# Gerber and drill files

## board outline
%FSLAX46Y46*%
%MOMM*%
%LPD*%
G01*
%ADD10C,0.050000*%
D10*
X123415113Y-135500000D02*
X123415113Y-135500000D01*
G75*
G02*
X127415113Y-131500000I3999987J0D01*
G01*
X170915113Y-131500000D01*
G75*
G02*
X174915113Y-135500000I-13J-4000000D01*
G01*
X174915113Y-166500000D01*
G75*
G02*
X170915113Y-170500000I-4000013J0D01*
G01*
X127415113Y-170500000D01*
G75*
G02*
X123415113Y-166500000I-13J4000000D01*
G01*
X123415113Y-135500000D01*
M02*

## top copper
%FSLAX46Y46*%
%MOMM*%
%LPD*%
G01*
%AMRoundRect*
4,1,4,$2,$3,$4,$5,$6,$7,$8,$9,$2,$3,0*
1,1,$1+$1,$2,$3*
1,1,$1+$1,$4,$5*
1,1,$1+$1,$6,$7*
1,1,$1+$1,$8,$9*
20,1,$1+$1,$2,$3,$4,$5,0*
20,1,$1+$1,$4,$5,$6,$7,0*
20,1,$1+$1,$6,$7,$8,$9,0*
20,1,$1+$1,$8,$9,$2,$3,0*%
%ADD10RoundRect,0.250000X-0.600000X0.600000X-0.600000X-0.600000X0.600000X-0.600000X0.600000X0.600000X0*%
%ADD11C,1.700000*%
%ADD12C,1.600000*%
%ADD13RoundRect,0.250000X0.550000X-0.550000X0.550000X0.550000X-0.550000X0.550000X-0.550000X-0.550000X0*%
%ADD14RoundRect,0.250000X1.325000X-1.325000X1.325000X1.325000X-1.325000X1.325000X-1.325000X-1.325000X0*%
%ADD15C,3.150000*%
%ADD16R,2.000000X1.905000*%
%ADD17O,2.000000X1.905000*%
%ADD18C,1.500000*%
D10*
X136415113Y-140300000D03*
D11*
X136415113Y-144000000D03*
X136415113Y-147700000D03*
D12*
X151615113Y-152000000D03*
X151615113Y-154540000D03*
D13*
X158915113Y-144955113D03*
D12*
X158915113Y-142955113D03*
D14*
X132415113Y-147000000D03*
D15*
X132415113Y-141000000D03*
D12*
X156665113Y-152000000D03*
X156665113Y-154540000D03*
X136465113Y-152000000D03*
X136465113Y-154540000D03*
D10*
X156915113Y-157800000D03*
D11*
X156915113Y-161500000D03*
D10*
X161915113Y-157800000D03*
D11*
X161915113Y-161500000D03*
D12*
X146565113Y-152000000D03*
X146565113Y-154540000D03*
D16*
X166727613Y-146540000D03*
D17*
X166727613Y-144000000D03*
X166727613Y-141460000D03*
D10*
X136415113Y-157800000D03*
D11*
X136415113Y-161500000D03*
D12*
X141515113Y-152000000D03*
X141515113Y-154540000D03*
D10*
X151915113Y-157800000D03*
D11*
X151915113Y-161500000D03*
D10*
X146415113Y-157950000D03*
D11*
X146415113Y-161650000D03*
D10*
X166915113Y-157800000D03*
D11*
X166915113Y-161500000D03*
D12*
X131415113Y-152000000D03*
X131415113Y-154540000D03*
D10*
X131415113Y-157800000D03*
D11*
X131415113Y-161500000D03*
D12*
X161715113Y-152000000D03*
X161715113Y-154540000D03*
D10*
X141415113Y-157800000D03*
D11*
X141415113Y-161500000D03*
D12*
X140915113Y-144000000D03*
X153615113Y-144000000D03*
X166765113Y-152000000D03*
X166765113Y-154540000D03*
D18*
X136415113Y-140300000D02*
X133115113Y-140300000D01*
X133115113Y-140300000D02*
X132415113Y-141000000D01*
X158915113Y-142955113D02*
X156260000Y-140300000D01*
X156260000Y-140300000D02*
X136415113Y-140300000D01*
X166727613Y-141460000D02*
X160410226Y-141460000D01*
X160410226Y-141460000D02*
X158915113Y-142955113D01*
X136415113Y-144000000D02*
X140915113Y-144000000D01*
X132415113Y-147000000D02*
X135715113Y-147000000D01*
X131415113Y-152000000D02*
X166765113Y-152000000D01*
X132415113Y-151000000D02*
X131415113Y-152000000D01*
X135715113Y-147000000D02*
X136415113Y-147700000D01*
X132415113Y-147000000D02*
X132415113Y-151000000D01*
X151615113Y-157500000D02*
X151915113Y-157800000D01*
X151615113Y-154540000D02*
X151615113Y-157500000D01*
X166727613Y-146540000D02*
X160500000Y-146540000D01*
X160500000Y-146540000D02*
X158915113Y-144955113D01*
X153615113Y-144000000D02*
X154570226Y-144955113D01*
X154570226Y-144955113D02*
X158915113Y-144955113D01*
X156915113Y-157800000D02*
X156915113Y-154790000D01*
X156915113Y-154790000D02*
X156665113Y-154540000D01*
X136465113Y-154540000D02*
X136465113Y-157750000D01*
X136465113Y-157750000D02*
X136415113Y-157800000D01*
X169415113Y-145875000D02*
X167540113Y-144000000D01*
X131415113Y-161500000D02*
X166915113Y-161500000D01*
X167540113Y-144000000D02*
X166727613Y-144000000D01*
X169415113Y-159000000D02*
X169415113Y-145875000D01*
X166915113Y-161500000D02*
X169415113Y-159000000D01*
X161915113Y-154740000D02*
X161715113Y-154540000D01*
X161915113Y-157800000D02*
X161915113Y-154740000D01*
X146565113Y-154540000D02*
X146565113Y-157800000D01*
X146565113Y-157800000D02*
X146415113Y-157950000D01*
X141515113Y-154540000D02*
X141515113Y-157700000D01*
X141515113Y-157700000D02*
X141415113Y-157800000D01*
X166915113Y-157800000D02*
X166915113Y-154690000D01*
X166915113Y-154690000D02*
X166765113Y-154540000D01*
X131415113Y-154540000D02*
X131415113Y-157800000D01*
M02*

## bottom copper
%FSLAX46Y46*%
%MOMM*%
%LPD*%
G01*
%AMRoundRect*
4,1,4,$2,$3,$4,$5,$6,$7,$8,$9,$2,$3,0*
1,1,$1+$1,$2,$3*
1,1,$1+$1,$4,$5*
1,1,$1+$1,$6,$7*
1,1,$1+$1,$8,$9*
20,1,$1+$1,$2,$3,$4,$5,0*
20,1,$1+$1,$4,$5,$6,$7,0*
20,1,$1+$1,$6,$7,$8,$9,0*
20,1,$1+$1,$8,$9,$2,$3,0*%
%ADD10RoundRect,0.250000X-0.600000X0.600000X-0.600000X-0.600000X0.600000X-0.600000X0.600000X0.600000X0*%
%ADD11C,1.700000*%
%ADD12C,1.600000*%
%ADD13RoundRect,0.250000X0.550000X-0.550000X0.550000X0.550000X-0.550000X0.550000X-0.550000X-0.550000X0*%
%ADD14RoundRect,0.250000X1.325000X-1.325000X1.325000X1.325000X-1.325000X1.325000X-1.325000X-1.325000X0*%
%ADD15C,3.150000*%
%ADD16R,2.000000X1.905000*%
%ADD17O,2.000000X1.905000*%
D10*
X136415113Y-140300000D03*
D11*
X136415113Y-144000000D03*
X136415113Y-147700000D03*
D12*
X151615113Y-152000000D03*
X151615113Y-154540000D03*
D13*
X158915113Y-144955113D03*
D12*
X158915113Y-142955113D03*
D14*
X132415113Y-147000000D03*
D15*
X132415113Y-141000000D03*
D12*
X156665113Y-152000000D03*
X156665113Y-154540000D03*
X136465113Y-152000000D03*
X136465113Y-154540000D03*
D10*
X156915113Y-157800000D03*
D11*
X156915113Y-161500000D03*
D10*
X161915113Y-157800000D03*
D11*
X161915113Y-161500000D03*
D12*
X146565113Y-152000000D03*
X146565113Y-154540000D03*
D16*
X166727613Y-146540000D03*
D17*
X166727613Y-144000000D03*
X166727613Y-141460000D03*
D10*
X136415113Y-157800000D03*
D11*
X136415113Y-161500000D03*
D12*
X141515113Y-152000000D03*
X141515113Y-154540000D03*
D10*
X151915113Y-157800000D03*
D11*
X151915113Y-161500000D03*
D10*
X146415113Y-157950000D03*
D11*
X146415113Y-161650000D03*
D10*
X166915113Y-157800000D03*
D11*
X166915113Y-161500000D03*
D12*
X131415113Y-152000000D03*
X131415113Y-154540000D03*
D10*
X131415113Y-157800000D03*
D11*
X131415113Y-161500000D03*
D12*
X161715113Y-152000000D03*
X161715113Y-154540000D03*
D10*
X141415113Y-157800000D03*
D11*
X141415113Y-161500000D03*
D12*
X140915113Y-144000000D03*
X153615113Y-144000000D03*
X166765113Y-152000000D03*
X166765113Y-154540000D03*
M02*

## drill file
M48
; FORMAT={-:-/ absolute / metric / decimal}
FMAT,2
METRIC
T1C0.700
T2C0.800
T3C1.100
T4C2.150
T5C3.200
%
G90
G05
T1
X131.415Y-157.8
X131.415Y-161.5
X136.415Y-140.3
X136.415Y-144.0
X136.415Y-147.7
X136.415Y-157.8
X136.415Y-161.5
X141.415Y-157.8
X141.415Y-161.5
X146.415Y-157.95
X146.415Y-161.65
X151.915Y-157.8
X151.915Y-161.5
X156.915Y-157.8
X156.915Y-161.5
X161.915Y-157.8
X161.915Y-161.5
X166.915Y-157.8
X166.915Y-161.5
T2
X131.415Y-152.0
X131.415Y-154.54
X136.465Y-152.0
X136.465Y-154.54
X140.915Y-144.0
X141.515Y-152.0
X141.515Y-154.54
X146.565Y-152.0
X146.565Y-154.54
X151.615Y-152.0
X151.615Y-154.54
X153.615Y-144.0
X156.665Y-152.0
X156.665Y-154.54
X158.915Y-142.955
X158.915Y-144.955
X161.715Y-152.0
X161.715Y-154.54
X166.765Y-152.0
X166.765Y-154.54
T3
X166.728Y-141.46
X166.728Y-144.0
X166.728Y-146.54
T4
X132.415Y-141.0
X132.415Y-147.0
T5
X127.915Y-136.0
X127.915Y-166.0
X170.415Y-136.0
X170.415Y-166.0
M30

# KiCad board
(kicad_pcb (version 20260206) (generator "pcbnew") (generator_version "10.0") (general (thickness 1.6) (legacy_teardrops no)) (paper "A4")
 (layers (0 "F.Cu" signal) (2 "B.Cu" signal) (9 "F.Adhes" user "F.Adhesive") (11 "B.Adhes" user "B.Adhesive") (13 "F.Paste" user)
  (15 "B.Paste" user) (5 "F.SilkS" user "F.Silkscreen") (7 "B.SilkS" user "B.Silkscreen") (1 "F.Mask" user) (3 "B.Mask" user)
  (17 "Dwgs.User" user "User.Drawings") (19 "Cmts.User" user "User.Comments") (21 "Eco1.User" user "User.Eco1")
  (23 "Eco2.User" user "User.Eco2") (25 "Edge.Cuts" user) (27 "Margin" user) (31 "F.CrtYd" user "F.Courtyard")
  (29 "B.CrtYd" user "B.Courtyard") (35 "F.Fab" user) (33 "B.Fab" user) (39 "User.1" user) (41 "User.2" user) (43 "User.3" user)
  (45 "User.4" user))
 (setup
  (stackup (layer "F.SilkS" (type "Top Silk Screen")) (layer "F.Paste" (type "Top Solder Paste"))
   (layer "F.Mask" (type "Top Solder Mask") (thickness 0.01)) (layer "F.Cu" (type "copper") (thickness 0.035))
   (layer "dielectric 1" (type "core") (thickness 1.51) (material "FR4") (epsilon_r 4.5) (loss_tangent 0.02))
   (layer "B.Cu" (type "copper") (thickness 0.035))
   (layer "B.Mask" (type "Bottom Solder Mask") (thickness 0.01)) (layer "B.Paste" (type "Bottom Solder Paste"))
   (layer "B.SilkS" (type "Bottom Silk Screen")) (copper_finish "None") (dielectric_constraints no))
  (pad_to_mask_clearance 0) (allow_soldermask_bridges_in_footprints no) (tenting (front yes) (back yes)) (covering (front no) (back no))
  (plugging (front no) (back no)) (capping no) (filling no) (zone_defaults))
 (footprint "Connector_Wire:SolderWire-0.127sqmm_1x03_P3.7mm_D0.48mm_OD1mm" (layer "F.Cu") (at 136.415113 140.3 -90)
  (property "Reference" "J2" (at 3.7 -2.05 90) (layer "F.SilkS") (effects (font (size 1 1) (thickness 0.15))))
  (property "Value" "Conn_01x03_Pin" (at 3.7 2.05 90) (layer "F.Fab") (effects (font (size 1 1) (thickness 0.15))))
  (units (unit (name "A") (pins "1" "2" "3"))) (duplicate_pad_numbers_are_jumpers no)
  (pad "1" thru_hole roundrect (at 0 0 270) (size 1.7 1.7) (drill 0.7) (layers "*.Cu" "*.Mask") (remove_unused_layers no)
   (roundrect_rratio 0.147059) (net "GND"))
  (pad "2" thru_hole circle (at 3.7 0 270) (size 1.7 1.7) (drill 0.7) (layers "*.Cu" "*.Mask") (remove_unused_layers no)
   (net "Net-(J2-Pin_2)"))
  (pad "3" thru_hole circle (at 7.4 0 270) (size 1.7 1.7) (drill 0.7) (layers "*.Cu" "*.Mask") (remove_unused_layers no) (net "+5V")))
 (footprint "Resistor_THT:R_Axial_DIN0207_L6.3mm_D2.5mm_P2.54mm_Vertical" (layer "F.Cu") (at 151.615113 152 -90)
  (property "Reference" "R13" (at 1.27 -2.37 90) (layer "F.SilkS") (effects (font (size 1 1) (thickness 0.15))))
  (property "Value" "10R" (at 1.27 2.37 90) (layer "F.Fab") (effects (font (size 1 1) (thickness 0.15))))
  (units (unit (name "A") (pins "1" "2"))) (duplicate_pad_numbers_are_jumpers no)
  (pad "1" thru_hole circle (at 0 0 270) (size 1.6 1.6) (drill 0.8) (layers "*.Cu" "*.Mask") (remove_unused_layers no) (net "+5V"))
  (pad "2" thru_hole circle (at 2.54 0 270) (size 1.6 1.6) (drill 0.8) (layers "*.Cu" "*.Mask") (remove_unused_layers no)
   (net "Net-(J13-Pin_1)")))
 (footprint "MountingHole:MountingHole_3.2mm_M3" (layer "F.Cu") (at 170.415113 136)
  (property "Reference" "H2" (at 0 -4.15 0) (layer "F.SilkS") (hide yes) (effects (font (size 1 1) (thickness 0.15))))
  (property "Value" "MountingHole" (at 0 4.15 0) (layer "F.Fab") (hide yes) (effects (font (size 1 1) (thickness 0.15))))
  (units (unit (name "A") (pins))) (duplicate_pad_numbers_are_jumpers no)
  (pad "" np_thru_hole circle (at 0 0) (size 3.2 3.2) (drill 3.2) (layers "*.Cu" "*.Mask")))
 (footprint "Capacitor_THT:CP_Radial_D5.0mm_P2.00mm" (layer "F.Cu") (at 158.915113 144.955113 90)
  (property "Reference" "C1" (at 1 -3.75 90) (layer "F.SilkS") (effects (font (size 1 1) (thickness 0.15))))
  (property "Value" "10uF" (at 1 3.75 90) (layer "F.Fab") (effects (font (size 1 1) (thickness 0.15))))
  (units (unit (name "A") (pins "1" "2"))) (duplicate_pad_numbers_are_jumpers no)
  (pad "1" thru_hole roundrect (at 0 0 90) (size 1.6 1.6) (drill 0.8) (layers "*.Cu" "*.Mask") (remove_unused_layers no)
   (roundrect_rratio 0.15625) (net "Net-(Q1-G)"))
  (pad "2" thru_hole circle (at 2 0 90) (size 1.6 1.6) (drill 0.8) (layers "*.Cu" "*.Mask") (remove_unused_layers no) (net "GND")))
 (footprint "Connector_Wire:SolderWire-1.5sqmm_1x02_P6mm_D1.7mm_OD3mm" (layer "F.Cu") (at 132.415113 147 90)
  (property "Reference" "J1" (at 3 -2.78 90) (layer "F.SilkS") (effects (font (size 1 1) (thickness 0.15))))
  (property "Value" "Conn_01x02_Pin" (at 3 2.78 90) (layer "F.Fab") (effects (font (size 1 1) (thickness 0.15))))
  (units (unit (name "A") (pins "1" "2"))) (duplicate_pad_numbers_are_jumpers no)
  (pad "1" thru_hole roundrect (at 0 0 90) (size 3.15 3.15) (drill 2.15) (layers "*.Cu" "*.Mask") (remove_unused_layers no)
   (roundrect_rratio 0.079365) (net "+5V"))
  (pad "2" thru_hole circle (at 6 0 90) (size 3.15 3.15) (drill 2.15) (layers "*.Cu" "*.Mask") (remove_unused_layers no) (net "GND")))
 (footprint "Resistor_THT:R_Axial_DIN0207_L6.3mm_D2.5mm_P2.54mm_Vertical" (layer "F.Cu") (at 156.665113 152 -90)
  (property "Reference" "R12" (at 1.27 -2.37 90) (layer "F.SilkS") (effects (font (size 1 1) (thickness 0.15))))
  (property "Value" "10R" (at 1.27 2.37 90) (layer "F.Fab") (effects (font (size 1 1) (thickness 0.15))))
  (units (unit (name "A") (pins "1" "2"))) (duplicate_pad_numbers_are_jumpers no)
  (pad "1" thru_hole circle (at 0 0 270) (size 1.6 1.6) (drill 0.8) (layers "*.Cu" "*.Mask") (remove_unused_layers no) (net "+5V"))
  (pad "2" thru_hole circle (at 2.54 0 270) (size 1.6 1.6) (drill 0.8) (layers "*.Cu" "*.Mask") (remove_unused_layers no)
   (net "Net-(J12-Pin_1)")))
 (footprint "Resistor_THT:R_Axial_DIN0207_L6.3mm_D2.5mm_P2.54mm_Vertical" (layer "F.Cu") (at 136.465113 152 -90)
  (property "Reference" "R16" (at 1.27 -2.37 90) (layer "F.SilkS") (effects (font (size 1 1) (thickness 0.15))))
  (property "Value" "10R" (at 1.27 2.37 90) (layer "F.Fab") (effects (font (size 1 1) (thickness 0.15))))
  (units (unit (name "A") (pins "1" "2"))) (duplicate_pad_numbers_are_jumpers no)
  (pad "1" thru_hole circle (at 0 0 270) (size 1.6 1.6) (drill 0.8) (layers "*.Cu" "*.Mask") (remove_unused_layers no) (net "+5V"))
  (pad "2" thru_hole circle (at 2.54 0 270) (size 1.6 1.6) (drill 0.8) (layers "*.Cu" "*.Mask") (remove_unused_layers no)
   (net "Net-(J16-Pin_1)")))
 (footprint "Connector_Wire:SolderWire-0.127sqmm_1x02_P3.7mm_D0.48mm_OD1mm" (layer "F.Cu") (at 156.915113 157.8 -90)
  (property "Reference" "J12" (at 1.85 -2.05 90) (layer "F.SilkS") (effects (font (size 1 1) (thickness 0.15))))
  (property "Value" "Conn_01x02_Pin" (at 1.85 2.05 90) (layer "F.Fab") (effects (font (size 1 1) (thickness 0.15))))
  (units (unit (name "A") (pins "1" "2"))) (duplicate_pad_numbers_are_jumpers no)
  (pad "1" thru_hole roundrect (at 0 0 270) (size 1.7 1.7) (drill 0.7) (layers "*.Cu" "*.Mask") (remove_unused_layers no)
   (roundrect_rratio 0.147059) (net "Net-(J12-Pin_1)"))
  (pad "2" thru_hole circle (at 3.7 0 270) (size 1.7 1.7) (drill 0.7) (layers "*.Cu" "*.Mask") (remove_unused_layers no)
   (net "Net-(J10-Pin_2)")))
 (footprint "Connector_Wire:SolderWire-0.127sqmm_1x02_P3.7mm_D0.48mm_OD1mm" (layer "F.Cu") (at 161.915113 157.8 -90)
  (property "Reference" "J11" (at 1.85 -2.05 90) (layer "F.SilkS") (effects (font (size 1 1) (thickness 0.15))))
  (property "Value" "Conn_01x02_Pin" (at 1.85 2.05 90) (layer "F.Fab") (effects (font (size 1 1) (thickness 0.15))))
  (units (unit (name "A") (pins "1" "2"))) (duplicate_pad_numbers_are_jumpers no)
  (pad "1" thru_hole roundrect (at 0 0 270) (size 1.7 1.7) (drill 0.7) (layers "*.Cu" "*.Mask") (remove_unused_layers no)
   (roundrect_rratio 0.147059) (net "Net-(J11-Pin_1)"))
  (pad "2" thru_hole circle (at 3.7 0 270) (size 1.7 1.7) (drill 0.7) (layers "*.Cu" "*.Mask") (remove_unused_layers no)
   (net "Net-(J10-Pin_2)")))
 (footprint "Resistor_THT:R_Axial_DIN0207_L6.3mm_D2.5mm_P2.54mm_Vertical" (layer "F.Cu") (at 146.565113 152 -90)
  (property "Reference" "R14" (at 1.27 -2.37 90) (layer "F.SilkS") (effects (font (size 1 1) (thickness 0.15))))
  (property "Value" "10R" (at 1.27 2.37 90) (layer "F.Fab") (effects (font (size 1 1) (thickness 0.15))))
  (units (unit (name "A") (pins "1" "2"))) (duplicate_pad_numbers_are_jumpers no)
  (pad "1" thru_hole circle (at 0 0 270) (size 1.6 1.6) (drill 0.8) (layers "*.Cu" "*.Mask") (remove_unused_layers no) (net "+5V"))
  (pad "2" thru_hole circle (at 2.54 0 270) (size 1.6 1.6) (drill 0.8) (layers "*.Cu" "*.Mask") (remove_unused_layers no)
   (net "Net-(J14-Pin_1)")))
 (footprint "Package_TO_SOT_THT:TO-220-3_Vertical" (layer "F.Cu") (at 166.727613 146.54 90)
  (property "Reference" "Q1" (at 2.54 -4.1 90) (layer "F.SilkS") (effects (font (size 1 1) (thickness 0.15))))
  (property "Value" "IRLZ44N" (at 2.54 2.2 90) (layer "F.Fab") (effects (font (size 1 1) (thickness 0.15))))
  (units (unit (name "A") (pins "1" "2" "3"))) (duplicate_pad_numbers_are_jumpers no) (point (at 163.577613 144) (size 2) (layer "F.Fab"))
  (pad "1" thru_hole rect (at 0 0 90) (size 1.905 2) (drill 1.1) (layers "*.Cu" "*.Mask") (remove_unused_layers no) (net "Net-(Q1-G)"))
  (pad "2" thru_hole oval (at 2.54 0 90) (size 1.905 2) (drill 1.1) (layers "*.Cu" "*.Mask") (remove_unused_layers no)
   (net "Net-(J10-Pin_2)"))
  (pad "3" thru_hole oval (at 5.08 0 90) (size 1.905 2) (drill 1.1) (layers "*.Cu" "*.Mask") (remove_unused_layers no) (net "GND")))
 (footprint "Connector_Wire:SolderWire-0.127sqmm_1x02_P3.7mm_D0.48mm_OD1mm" (layer "F.Cu") (at 136.415113 157.8 -90)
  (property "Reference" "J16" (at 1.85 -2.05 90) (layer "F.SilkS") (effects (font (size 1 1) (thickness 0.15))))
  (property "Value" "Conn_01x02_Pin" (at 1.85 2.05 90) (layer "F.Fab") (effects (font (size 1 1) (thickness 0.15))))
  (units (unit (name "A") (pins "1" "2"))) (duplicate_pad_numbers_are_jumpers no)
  (pad "1" thru_hole roundrect (at 0 0 270) (size 1.7 1.7) (drill 0.7) (layers "*.Cu" "*.Mask") (remove_unused_layers no)
   (roundrect_rratio 0.147059) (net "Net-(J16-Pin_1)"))
  (pad "2" thru_hole circle (at 3.7 0 270) (size 1.7 1.7) (drill 0.7) (layers "*.Cu" "*.Mask") (remove_unused_layers no)
   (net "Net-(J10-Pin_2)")))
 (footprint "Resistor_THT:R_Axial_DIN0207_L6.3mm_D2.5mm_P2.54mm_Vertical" (layer "F.Cu") (at 141.515113 152 -90)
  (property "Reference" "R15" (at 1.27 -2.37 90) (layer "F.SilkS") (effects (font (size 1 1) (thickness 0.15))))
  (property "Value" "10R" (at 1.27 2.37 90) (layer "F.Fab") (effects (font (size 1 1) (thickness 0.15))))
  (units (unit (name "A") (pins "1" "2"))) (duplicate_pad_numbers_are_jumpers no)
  (pad "1" thru_hole circle (at 0 0 270) (size 1.6 1.6) (drill 0.8) (layers "*.Cu" "*.Mask") (remove_unused_layers no) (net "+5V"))
  (pad "2" thru_hole circle (at 2.54 0 270) (size 1.6 1.6) (drill 0.8) (layers "*.Cu" "*.Mask") (remove_unused_layers no)
   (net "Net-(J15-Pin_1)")))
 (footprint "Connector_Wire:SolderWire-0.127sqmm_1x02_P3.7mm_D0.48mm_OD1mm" (layer "F.Cu") (at 151.915113 157.8 -90)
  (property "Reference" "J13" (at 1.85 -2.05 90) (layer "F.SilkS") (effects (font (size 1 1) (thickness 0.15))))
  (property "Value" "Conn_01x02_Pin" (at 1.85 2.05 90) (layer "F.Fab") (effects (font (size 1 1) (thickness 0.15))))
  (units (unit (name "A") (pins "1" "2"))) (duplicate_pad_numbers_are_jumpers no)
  (pad "1" thru_hole roundrect (at 0 0 270) (size 1.7 1.7) (drill 0.7) (layers "*.Cu" "*.Mask") (remove_unused_layers no)
   (roundrect_rratio 0.147059) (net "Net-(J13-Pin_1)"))
  (pad "2" thru_hole circle (at 3.7 0 270) (size 1.7 1.7) (drill 0.7) (layers "*.Cu" "*.Mask") (remove_unused_layers no)
   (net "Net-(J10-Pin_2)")))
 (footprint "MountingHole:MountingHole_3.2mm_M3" (layer "F.Cu") (at 127.915113 136)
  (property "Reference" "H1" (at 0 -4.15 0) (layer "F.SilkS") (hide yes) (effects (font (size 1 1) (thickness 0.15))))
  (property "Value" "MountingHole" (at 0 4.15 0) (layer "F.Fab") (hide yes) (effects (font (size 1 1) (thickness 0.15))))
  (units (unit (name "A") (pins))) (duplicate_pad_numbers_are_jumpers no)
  (pad "" np_thru_hole circle (at 0 0) (size 3.2 3.2) (drill 3.2) (layers "*.Cu" "*.Mask")))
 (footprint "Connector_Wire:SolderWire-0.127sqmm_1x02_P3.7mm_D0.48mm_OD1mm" (layer "F.Cu") (at 146.415113 157.95 -90)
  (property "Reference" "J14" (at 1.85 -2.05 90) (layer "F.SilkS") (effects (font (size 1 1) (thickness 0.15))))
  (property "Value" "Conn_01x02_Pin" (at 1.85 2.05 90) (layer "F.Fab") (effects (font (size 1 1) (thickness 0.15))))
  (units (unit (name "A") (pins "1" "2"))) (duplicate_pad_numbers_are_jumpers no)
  (pad "1" thru_hole roundrect (at 0 0 270) (size 1.7 1.7) (drill 0.7) (layers "*.Cu" "*.Mask") (remove_unused_layers no)
   (roundrect_rratio 0.147059) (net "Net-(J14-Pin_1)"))
  (pad "2" thru_hole circle (at 3.7 0 270) (size 1.7 1.7) (drill 0.7) (layers "*.Cu" "*.Mask") (remove_unused_layers no)
   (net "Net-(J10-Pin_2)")))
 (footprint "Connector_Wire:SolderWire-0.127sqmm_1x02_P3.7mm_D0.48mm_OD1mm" (layer "F.Cu") (at 166.915113 157.8 -90)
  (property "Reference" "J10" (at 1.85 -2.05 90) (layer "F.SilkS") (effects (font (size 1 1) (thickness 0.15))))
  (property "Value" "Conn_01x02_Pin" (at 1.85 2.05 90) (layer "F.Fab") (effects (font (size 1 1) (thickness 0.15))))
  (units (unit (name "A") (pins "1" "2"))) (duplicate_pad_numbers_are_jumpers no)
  (pad "1" thru_hole roundrect (at 0 0 270) (size 1.7 1.7) (drill 0.7) (layers "*.Cu" "*.Mask") (remove_unused_layers no)
   (roundrect_rratio 0.147059) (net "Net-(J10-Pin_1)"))
  (pad "2" thru_hole circle (at 3.7 0 270) (size 1.7 1.7) (drill 0.7) (layers "*.Cu" "*.Mask") (remove_unused_layers no)
   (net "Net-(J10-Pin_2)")))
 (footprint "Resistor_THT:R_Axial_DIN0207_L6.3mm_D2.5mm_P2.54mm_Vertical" (layer "F.Cu") (at 131.415113 152 -90)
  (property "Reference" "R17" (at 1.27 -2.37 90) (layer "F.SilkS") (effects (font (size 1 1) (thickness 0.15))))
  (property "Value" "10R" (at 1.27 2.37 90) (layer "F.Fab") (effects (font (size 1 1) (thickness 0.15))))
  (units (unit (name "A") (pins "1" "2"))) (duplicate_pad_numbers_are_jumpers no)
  (pad "1" thru_hole circle (at 0 0 270) (size 1.6 1.6) (drill 0.8) (layers "*.Cu" "*.Mask") (remove_unused_layers no) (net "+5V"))
  (pad "2" thru_hole circle (at 2.54 0 270) (size 1.6 1.6) (drill 0.8) (layers "*.Cu" "*.Mask") (remove_unused_layers no)
   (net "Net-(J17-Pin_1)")))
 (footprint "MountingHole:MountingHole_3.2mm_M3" (layer "F.Cu") (at 127.915113 166)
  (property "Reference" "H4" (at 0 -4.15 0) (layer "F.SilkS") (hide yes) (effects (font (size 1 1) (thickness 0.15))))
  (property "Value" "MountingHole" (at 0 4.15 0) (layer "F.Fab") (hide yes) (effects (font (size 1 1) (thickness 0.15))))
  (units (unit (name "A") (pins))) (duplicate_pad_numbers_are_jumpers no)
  (pad "" np_thru_hole circle (at 0 0) (size 3.2 3.2) (drill 3.2) (layers "*.Cu" "*.Mask")))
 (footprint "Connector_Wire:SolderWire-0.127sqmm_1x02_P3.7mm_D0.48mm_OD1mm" (layer "F.Cu") (at 131.415113 157.8 -90)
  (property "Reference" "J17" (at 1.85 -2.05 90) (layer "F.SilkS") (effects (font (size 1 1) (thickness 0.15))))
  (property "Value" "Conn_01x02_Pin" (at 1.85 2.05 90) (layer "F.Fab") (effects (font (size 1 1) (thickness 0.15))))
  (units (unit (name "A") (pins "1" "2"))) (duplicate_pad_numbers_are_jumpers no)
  (pad "1" thru_hole roundrect (at 0 0 270) (size 1.7 1.7) (drill 0.7) (layers "*.Cu" "*.Mask") (remove_unused_layers no)
   (roundrect_rratio 0.147059) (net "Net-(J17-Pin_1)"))
  (pad "2" thru_hole circle (at 3.7 0 270) (size 1.7 1.7) (drill 0.7) (layers "*.Cu" "*.Mask") (remove_unused_layers no)
   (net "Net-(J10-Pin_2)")))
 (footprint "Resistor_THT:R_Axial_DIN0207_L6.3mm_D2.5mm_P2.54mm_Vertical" (layer "F.Cu") (at 161.715113 152 -90)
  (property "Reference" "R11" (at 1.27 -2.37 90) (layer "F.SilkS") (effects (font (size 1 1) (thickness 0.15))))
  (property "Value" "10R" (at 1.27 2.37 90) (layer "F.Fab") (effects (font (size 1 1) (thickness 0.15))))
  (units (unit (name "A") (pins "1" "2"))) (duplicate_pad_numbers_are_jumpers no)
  (pad "1" thru_hole circle (at 0 0 270) (size 1.6 1.6) (drill 0.8) (layers "*.Cu" "*.Mask") (remove_unused_layers no) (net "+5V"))
  (pad "2" thru_hole circle (at 2.54 0 270) (size 1.6 1.6) (drill 0.8) (layers "*.Cu" "*.Mask") (remove_unused_layers no)
   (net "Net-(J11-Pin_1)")))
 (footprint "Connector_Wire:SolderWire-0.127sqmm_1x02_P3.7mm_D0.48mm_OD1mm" (layer "F.Cu") (at 141.415113 157.8 -90)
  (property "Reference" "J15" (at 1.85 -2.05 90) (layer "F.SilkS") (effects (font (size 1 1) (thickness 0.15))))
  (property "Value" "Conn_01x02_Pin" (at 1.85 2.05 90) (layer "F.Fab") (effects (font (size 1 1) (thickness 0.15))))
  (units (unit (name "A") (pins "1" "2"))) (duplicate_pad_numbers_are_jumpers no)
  (pad "1" thru_hole roundrect (at 0 0 270) (size 1.7 1.7) (drill 0.7) (layers "*.Cu" "*.Mask") (remove_unused_layers no)
   (roundrect_rratio 0.147059) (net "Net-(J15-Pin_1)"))
  (pad "2" thru_hole circle (at 3.7 0 270) (size 1.7 1.7) (drill 0.7) (layers "*.Cu" "*.Mask") (remove_unused_layers no)
   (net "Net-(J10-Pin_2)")))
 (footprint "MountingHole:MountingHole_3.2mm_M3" (layer "F.Cu") (at 170.415113 166)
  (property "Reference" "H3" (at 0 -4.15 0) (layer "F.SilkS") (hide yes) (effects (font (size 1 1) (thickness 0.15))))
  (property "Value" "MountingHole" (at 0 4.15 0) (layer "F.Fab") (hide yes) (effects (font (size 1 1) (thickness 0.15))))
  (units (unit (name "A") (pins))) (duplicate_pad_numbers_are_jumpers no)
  (pad "" np_thru_hole circle (at 0 0) (size 3.2 3.2) (drill 3.2) (layers "*.Cu" "*.Mask")))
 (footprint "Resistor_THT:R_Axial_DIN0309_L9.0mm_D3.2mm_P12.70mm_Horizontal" (layer "F.Cu") (at 140.915113 144)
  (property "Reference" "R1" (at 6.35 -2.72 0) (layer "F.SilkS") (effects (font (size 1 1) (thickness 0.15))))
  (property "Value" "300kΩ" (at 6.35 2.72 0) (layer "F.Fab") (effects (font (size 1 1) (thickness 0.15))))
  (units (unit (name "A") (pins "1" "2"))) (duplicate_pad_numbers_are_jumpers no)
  (pad "1" thru_hole circle (at 0 0) (size 1.6 1.6) (drill 0.8) (layers "*.Cu" "*.Mask") (remove_unused_layers no) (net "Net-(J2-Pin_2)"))
  (pad "2" thru_hole circle (at 12.7 0) (size 1.6 1.6) (drill 0.8) (layers "*.Cu" "*.Mask") (remove_unused_layers no) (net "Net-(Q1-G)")))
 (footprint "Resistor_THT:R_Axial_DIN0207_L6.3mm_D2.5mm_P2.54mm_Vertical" (layer "F.Cu") (at 166.765113 152 -90)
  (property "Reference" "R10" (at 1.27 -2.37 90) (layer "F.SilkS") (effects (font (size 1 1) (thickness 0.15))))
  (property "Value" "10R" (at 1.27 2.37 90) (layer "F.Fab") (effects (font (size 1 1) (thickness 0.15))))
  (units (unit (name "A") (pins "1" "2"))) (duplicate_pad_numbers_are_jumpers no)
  (pad "1" thru_hole circle (at 0 0 270) (size 1.6 1.6) (drill 0.8) (layers "*.Cu" "*.Mask") (remove_unused_layers no) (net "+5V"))
  (pad "2" thru_hole circle (at 2.54 0 270) (size 1.6 1.6) (drill 0.8) (layers "*.Cu" "*.Mask") (remove_unused_layers no)
   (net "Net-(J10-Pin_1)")))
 (gr_rect (start 123.415113 131.5) (end 174.915113 170.5) (radius 4) (stroke (width 0.05) (type solid)) (fill no) (layer "Edge.Cuts"))
 (segment (start 136.415113 140.3) (end 133.115113 140.3) (width 1.5) (layer "F.Cu") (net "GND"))
 (segment (start 133.115113 140.3) (end 132.415113 141) (width 1.5) (layer "F.Cu") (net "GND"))
 (segment (start 158.915113 142.955113) (end 156.26 140.3) (width 1.5) (layer "F.Cu") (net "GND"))
 (segment (start 156.26 140.3) (end 136.415113 140.3) (width 1.5) (layer "F.Cu") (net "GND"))
 (segment (start 166.727613 141.46) (end 160.410226 141.46) (width 1.5) (layer "F.Cu") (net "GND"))
 (segment (start 160.410226 141.46) (end 158.915113 142.955113) (width 1.5) (layer "F.Cu") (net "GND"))
 (segment (start 136.415113 144) (end 140.915113 144) (width 1.5) (layer "F.Cu") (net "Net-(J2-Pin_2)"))
 (segment (start 132.415113 147) (end 135.715113 147) (width 1.5) (layer "F.Cu") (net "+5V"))
 (segment (start 131.415113 152) (end 166.765113 152) (width 1.5) (layer "F.Cu") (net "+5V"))
 (segment (start 132.415113 151) (end 131.415113 152) (width 1.5) (layer "F.Cu") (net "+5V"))
 (segment (start 135.715113 147) (end 136.415113 147.7) (width 1.5) (layer "F.Cu") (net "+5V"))
 (segment (start 132.415113 147) (end 132.415113 151) (width 1.5) (layer "F.Cu") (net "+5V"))
 (segment (start 151.615113 157.5) (end 151.915113 157.8) (width 1.5) (layer "F.Cu") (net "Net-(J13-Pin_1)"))
 (segment (start 151.615113 154.54) (end 151.615113 157.5) (width 1.5) (layer "F.Cu") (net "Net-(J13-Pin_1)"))
 (segment (start 166.727613 146.54) (end 160.5 146.54) (width 1.5) (layer "F.Cu") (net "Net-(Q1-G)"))
 (segment (start 160.5 146.54) (end 158.915113 144.955113) (width 1.5) (layer "F.Cu") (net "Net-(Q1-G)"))
 (segment (start 153.615113 144) (end 154.570226 144.955113) (width 1.5) (layer "F.Cu") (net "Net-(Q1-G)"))
 (segment (start 154.570226 144.955113) (end 158.915113 144.955113) (width 1.5) (layer "F.Cu") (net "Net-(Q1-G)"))
 (segment (start 156.915113 157.8) (end 156.915113 154.79) (width 1.5) (layer "F.Cu") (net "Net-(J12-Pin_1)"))
 (segment (start 156.915113 154.79) (end 156.665113 154.54) (width 1.5) (layer "F.Cu") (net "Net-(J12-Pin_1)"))
 (segment (start 136.465113 154.54) (end 136.465113 157.75) (width 1.5) (layer "F.Cu") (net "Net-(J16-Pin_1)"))
 (segment (start 136.465113 157.75) (end 136.415113 157.8) (width 1.5) (layer "F.Cu") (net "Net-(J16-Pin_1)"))
 (segment (start 169.415113 145.875) (end 167.540113 144) (width 1.5) (layer "F.Cu") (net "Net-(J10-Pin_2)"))
 (segment (start 131.415113 161.5) (end 166.915113 161.5) (width 1.5) (layer "F.Cu") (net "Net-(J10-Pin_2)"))
 (segment (start 167.540113 144) (end 166.727613 144) (width 1.5) (layer "F.Cu") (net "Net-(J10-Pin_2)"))
 (segment (start 169.415113 159) (end 169.415113 145.875) (width 1.5) (layer "F.Cu") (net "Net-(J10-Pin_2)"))
 (segment (start 166.915113 161.5) (end 169.415113 159) (width 1.5) (layer "F.Cu") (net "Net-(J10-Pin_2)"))
 (segment (start 161.915113 154.74) (end 161.715113 154.54) (width 1.5) (layer "F.Cu") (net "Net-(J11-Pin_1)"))
 (segment (start 161.915113 157.8) (end 161.915113 154.74) (width 1.5) (layer "F.Cu") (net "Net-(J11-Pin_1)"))
 (segment (start 146.565113 154.54) (end 146.565113 157.8) (width 1.5) (layer "F.Cu") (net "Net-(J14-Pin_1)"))
 (segment (start 146.565113 157.8) (end 146.415113 157.95) (width 1.5) (layer "F.Cu") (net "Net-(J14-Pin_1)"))
 (segment (start 141.515113 154.54) (end 141.515113 157.7) (width 1.5) (layer "F.Cu") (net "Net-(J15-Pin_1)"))
 (segment (start 141.515113 157.7) (end 141.415113 157.8) (width 1.5) (layer "F.Cu") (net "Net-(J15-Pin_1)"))
 (segment (start 166.915113 157.8) (end 166.915113 154.69) (width 1.5) (layer "F.Cu") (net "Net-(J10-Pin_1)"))
 (segment (start 166.915113 154.69) (end 166.765113 154.54) (width 1.5) (layer "F.Cu") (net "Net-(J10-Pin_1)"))
 (segment (start 131.415113 154.54) (end 131.415113 157.8) (width 1.5) (layer "F.Cu") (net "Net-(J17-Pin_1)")))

